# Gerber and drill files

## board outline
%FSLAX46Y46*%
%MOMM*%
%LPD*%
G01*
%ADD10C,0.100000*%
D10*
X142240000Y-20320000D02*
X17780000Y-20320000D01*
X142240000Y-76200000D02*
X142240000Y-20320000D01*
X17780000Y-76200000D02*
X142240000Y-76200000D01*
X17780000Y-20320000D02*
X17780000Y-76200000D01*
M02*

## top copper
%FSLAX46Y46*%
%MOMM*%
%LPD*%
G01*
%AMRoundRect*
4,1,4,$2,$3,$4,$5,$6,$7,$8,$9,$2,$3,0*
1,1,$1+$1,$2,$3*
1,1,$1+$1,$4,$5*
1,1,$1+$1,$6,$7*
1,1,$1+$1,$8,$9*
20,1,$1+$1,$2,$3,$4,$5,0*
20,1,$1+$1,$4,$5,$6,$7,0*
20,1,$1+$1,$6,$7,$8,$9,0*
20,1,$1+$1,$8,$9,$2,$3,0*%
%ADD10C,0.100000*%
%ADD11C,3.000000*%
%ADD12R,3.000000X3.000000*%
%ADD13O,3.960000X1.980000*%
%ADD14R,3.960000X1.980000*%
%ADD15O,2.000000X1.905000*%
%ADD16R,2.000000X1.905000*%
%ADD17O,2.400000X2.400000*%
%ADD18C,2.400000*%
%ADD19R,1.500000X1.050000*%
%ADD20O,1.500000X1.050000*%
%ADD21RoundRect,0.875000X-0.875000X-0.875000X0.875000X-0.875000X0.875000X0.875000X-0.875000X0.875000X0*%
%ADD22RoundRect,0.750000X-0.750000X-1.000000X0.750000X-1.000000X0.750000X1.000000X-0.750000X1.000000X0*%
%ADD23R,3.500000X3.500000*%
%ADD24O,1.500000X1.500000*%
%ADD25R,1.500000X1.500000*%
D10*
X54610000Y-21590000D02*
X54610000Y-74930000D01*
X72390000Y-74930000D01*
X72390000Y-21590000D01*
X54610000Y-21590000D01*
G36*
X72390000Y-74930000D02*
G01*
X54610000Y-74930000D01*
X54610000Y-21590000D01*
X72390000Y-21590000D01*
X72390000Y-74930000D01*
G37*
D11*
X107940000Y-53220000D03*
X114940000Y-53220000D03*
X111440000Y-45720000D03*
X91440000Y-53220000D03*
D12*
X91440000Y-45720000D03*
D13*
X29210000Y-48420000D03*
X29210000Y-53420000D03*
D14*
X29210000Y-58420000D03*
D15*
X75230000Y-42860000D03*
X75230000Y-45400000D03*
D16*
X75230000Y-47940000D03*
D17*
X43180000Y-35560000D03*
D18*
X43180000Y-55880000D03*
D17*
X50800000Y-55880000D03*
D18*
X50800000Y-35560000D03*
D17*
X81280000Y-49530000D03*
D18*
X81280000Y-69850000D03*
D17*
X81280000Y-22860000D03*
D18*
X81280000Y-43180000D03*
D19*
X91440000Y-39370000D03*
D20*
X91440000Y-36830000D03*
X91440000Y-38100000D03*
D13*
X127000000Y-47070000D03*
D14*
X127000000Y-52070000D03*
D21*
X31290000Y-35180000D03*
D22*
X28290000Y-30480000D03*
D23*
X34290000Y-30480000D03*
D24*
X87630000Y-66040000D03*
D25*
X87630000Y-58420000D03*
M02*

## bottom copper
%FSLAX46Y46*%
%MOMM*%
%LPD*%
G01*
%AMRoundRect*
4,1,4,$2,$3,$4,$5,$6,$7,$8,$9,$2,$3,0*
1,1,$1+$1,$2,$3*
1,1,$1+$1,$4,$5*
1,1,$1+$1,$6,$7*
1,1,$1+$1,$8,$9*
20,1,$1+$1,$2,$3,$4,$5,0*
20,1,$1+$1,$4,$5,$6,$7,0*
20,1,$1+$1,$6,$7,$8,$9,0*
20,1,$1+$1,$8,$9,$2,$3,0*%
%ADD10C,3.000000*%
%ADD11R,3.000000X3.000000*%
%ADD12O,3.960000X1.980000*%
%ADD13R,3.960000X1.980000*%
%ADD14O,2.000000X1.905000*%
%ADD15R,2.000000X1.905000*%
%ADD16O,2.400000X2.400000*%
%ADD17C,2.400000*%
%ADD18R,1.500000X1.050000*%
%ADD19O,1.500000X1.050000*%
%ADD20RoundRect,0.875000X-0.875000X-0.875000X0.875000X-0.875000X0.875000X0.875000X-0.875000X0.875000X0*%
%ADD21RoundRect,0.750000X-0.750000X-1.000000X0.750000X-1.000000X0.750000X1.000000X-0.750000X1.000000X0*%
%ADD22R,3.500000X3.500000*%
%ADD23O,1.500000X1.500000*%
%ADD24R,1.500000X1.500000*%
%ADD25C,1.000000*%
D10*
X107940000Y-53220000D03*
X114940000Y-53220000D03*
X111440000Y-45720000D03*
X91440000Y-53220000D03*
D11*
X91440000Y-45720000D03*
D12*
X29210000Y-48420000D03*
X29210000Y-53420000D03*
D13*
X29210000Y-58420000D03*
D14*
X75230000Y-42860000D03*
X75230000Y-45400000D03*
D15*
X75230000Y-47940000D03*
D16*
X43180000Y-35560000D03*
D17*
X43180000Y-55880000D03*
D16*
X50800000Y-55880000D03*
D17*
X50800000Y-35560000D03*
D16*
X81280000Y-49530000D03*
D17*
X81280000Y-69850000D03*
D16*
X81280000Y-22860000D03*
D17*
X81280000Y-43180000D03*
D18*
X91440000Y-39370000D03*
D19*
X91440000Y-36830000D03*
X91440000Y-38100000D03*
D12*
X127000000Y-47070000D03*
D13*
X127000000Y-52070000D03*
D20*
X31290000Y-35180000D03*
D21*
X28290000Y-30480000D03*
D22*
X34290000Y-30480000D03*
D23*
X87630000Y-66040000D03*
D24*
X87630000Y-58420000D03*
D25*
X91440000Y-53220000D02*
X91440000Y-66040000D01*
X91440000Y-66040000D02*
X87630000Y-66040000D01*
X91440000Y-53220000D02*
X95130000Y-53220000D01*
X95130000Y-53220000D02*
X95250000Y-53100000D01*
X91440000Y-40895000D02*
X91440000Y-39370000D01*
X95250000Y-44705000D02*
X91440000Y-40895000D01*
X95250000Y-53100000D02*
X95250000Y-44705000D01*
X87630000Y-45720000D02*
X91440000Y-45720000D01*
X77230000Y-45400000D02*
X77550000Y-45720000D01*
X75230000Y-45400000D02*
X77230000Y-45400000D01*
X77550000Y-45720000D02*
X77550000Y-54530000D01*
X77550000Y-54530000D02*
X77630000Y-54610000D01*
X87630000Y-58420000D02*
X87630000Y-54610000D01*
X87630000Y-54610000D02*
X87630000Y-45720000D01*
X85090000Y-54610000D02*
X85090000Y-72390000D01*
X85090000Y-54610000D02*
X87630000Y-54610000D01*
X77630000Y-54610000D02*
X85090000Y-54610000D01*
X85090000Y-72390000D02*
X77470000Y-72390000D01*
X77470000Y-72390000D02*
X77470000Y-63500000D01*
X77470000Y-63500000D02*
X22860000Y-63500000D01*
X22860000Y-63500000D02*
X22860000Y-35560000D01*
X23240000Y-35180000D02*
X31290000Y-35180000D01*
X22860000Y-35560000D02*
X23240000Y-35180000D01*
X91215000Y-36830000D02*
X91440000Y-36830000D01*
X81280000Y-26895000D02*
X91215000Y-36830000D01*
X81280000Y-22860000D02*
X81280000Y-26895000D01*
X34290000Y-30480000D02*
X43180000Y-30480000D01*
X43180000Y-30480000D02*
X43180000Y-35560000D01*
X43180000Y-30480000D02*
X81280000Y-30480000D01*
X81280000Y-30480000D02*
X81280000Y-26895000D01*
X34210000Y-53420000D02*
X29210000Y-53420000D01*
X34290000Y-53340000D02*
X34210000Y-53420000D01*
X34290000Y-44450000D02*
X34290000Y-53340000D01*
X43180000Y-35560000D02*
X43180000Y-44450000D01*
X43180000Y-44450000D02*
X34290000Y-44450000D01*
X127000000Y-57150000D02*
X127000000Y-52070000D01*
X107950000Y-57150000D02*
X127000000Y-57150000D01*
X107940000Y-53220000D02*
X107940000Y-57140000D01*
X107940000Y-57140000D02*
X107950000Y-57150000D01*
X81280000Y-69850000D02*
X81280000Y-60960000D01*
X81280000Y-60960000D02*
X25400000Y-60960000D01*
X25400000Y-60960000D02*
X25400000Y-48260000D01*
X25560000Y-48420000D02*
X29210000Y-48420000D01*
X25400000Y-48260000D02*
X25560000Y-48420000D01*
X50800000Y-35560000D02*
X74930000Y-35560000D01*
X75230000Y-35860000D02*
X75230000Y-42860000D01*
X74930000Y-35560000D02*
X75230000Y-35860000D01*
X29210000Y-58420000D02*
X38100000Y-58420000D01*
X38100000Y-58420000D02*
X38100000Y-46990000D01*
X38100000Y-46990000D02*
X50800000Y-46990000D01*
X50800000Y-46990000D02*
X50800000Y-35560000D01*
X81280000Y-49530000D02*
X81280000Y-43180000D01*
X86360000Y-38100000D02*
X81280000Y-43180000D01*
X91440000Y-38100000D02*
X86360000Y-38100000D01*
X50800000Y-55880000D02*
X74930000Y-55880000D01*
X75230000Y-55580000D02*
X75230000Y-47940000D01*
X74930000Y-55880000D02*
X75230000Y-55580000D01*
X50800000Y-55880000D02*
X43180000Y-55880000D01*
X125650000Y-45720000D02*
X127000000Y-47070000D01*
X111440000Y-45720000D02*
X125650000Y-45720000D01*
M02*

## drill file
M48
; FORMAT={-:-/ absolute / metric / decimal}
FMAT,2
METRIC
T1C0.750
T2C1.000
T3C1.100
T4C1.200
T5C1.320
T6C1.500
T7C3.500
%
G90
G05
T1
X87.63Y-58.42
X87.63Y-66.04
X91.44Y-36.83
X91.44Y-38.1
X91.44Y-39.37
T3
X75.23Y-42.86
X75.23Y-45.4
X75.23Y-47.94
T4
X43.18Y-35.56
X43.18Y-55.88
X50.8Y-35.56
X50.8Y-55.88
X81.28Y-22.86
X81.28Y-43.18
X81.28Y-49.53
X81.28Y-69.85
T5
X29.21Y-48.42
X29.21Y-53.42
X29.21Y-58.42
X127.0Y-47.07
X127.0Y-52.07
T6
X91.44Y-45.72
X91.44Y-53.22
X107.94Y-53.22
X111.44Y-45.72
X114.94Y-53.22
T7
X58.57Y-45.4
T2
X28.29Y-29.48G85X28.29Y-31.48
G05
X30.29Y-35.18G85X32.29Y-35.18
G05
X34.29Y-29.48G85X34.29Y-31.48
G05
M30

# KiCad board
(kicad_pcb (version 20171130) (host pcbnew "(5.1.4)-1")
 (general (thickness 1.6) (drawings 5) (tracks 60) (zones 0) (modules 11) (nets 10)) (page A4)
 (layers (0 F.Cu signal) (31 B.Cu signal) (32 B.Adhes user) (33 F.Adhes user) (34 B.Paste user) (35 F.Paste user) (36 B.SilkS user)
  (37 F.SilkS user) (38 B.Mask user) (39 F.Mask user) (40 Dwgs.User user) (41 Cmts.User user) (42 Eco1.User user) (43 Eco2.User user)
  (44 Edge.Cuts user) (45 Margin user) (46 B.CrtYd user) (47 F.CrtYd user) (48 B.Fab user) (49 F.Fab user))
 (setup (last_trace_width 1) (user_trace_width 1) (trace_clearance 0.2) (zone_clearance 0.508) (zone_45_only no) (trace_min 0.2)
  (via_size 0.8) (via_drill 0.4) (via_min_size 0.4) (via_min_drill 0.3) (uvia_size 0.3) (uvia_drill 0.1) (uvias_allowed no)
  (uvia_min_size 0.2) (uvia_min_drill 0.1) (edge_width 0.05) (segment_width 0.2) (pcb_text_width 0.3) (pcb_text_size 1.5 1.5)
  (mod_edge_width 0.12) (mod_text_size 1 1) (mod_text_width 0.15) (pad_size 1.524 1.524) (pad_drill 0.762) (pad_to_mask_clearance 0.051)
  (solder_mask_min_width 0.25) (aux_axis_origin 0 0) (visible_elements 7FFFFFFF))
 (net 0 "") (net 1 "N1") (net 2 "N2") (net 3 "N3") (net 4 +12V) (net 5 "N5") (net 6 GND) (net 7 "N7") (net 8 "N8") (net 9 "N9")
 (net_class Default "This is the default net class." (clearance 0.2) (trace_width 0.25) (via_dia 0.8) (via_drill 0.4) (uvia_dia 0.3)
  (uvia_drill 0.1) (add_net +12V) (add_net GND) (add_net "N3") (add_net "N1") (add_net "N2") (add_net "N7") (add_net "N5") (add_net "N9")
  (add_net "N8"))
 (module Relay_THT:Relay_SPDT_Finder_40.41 (layer F.Cu) (at 91.44 45.72)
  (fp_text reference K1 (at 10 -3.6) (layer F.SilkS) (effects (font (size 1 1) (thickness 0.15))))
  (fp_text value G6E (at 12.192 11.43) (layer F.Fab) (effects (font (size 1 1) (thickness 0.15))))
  (pad 12 thru_hole circle (at 16.5 7.5) (size 3 3) (drill 1.5) (layers *.Cu *.Mask) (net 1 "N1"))
  (pad 14 thru_hole circle (at 23.5 7.5) (size 3 3) (drill 1.5) (layers *.Cu *.Mask))
  (pad 11 thru_hole circle (at 20 0) (size 3 3) (drill 1.5) (layers *.Cu *.Mask) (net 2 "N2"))
  (pad A2 thru_hole circle (at 0 7.5) (size 3 3) (drill 1.5) (layers *.Cu *.Mask) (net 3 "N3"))
  (pad A1 thru_hole rect (at 0 0) (size 3 3) (drill 1.5) (layers *.Cu *.Mask) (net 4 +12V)))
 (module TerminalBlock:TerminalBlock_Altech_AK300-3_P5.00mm (layer F.Cu) (at 29.21 58.42 90)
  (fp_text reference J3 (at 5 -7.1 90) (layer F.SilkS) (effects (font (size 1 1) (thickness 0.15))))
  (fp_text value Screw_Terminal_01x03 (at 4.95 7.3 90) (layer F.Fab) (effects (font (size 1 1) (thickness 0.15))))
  (pad 3 thru_hole oval (at 10 0 90) (size 1.98 3.96) (drill 1.32) (layers *.Cu *.Mask) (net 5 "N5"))
  (pad 2 thru_hole oval (at 5 0 90) (size 1.98 3.96) (drill 1.32) (layers *.Cu *.Mask) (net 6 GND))
  (pad 1 thru_hole rect (at 0 0 90) (size 1.98 3.96) (drill 1.32) (layers *.Cu *.Mask) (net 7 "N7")))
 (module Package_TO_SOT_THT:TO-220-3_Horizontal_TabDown (layer F.Cu) (at 75.23 47.94 90)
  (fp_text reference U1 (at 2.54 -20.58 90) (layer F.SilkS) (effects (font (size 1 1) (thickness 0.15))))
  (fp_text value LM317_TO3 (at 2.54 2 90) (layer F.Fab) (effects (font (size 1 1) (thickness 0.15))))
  (pad 3 thru_hole oval (at 5.08 0 90) (size 1.905 2) (drill 1.1) (layers *.Cu *.Mask) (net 7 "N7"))
  (pad 2 thru_hole oval (at 2.54 0 90) (size 1.905 2) (drill 1.1) (layers *.Cu *.Mask) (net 4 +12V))
  (pad 1 thru_hole rect (at 0 0 90) (size 1.905 2) (drill 1.1) (layers *.Cu *.Mask) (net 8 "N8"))
  (pad "" np_thru_hole oval (at 2.54 -16.66 90) (size 3.5 3.5) (drill 3.5) (layers *.Cu *.Mask)))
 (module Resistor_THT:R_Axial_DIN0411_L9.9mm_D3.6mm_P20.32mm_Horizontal (layer F.Cu) (at 43.18 55.88 90)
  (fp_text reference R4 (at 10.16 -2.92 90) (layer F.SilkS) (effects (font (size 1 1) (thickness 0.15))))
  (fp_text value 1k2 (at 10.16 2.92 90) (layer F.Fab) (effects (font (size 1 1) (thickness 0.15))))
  (pad 2 thru_hole oval (at 20.32 0 90) (size 2.4 2.4) (drill 1.2) (layers *.Cu *.Mask) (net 6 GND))
  (pad 1 thru_hole circle (at 0 0 90) (size 2.4 2.4) (drill 1.2) (layers *.Cu *.Mask) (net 8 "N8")))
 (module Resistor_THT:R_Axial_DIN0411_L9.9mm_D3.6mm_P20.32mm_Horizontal (layer F.Cu) (at 50.8 35.56 270)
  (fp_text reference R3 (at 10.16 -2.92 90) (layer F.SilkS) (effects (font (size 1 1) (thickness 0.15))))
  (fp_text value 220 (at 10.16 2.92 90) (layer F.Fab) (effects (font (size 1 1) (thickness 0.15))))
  (pad 2 thru_hole oval (at 20.32 0 270) (size 2.4 2.4) (drill 1.2) (layers *.Cu *.Mask) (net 8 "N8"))
  (pad 1 thru_hole circle (at 0 0 270) (size 2.4 2.4) (drill 1.2) (layers *.Cu *.Mask) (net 7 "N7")))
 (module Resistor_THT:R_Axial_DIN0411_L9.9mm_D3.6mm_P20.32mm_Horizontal (layer F.Cu) (at 81.28 69.85 90)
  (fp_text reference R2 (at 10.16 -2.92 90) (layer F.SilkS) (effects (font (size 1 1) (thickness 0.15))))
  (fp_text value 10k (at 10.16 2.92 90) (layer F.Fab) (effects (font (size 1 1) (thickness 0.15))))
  (pad 2 thru_hole oval (at 20.32 0 90) (size 2.4 2.4) (drill 1.2) (layers *.Cu *.Mask) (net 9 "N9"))
  (pad 1 thru_hole circle (at 0 0 90) (size 2.4 2.4) (drill 1.2) (layers *.Cu *.Mask) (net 5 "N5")))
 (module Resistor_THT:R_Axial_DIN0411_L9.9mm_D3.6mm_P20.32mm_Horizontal (layer F.Cu) (at 81.28 43.18 90)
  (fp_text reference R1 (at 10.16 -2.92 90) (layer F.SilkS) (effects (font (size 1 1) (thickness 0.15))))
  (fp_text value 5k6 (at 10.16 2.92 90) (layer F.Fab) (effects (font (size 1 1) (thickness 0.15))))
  (pad 2 thru_hole oval (at 20.32 0 90) (size 2.4 2.4) (drill 1.2) (layers *.Cu *.Mask) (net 6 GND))
  (pad 1 thru_hole circle (at 0 0 90) (size 2.4 2.4) (drill 1.2) (layers *.Cu *.Mask) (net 9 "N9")))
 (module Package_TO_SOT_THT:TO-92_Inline (layer F.Cu) (at 91.44 39.37 90)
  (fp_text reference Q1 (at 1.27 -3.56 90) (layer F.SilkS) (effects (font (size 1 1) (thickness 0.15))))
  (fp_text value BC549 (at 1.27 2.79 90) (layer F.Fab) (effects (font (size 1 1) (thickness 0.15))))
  (pad 1 thru_hole rect (at 0 0 90) (size 1.05 1.5) (drill 0.75) (layers *.Cu *.Mask) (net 3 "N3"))
  (pad 3 thru_hole oval (at 2.54 0 90) (size 1.05 1.5) (drill 0.75) (layers *.Cu *.Mask) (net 6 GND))
  (pad 2 thru_hole oval (at 1.27 0 90) (size 1.05 1.5) (drill 0.75) (layers *.Cu *.Mask) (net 9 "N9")))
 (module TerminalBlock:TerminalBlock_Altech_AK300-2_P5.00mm (layer F.Cu) (at 127 52.07 90)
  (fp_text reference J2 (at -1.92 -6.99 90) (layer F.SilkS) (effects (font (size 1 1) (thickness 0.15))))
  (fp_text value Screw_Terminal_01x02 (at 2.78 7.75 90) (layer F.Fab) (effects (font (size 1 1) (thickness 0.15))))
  (pad 2 thru_hole oval (at 5 0 90) (size 1.98 3.96) (drill 1.32) (layers *.Cu *.Mask) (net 2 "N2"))
  (pad 1 thru_hole rect (at 0 0 90) (size 1.98 3.96) (drill 1.32) (layers *.Cu *.Mask) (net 1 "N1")))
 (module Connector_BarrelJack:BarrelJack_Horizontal (layer F.Cu) (at 34.29 30.48)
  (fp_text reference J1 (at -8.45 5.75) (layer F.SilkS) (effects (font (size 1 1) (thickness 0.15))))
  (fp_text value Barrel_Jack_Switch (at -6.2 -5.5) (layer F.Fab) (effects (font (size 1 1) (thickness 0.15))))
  (pad 3 thru_hole roundrect (at -3 4.7) (size 3.5 3.5) (drill oval 3 1) (layers *.Cu *.Mask) (roundrect_rratio 0.25) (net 4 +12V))
  (pad 2 thru_hole roundrect (at -6 0) (size 3 3.5) (drill oval 1 3) (layers *.Cu *.Mask) (roundrect_rratio 0.25))
  (pad 1 thru_hole rect (at 0 0) (size 3.5 3.5) (drill oval 1 3) (layers *.Cu *.Mask) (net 6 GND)))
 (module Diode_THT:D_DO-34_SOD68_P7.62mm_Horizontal (layer F.Cu) (at 87.63 58.42 270)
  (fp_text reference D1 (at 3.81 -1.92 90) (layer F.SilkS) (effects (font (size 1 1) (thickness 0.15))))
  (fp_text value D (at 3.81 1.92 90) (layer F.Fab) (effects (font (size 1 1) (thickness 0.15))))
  (pad 2 thru_hole oval (at 7.62 0 270) (size 1.5 1.5) (drill 0.75) (layers *.Cu *.Mask) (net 3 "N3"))
  (pad 1 thru_hole rect (at 0 0 270) (size 1.5 1.5) (drill 0.75) (layers *.Cu *.Mask) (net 4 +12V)))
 (gr_poly (pts (xy 54.61 21.59) (xy 54.61 74.93) (xy 72.39 74.93) (xy 72.39 21.59)) (layer F.Cu) (width 0.1))
 (gr_line (start 142.24 20.32) (end 17.78 20.32) (layer Edge.Cuts) (width 0.1))
 (gr_line (start 142.24 76.2) (end 142.24 20.32) (layer Edge.Cuts) (width 0.1))
 (gr_line (start 17.78 76.2) (end 142.24 76.2) (layer Edge.Cuts) (width 0.1))
 (gr_line (start 17.78 20.32) (end 17.78 76.2) (layer Edge.Cuts) (width 0.1))
 (segment (start 91.44 53.22) (end 91.44 66.04) (width 1) (layer B.Cu) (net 3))
 (segment (start 91.44 66.04) (end 87.63 66.04) (width 1) (layer B.Cu) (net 3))
 (segment (start 91.44 53.22) (end 95.13 53.22) (width 1) (layer B.Cu) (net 3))
 (segment (start 95.13 53.22) (end 95.25 53.1) (width 1) (layer B.Cu) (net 3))
 (segment (start 91.44 40.895) (end 91.44 39.37) (width 1) (layer B.Cu) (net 3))
 (segment (start 95.25 44.705) (end 91.44 40.895) (width 1) (layer B.Cu) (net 3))
 (segment (start 95.25 53.1) (end 95.25 44.705) (width 1) (layer B.Cu) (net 3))
 (segment (start 87.63 45.72) (end 91.44 45.72) (width 1) (layer B.Cu) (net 4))
 (segment (start 77.23 45.4) (end 77.55 45.72) (width 1) (layer B.Cu) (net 4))
 (segment (start 75.23 45.4) (end 77.23 45.4) (width 1) (layer B.Cu) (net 4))
 (segment (start 77.55 45.72) (end 77.55 54.53) (width 1) (layer B.Cu) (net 4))
 (segment (start 77.55 54.53) (end 77.63 54.61) (width 1) (layer B.Cu) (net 4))
 (segment (start 87.63 58.42) (end 87.63 54.61) (width 1) (layer B.Cu) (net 4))
 (segment (start 87.63 54.61) (end 87.63 45.72) (width 1) (layer B.Cu) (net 4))
 (segment (start 85.09 54.61) (end 85.09 72.39) (width 1) (layer B.Cu) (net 4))
 (segment (start 85.09 54.61) (end 87.63 54.61) (width 1) (layer B.Cu) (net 4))
 (segment (start 77.63 54.61) (end 85.09 54.61) (width 1) (layer B.Cu) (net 4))
 (segment (start 85.09 72.39) (end 77.47 72.39) (width 1) (layer B.Cu) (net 4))
 (segment (start 77.47 72.39) (end 77.47 63.5) (width 1) (layer B.Cu) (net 4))
 (segment (start 77.47 63.5) (end 22.86 63.5) (width 1) (layer B.Cu) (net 4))
 (segment (start 22.86 63.5) (end 22.86 35.56) (width 1) (layer B.Cu) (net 4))
 (segment (start 23.24 35.18) (end 31.29 35.18) (width 1) (layer B.Cu) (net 4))
 (segment (start 22.86 35.56) (end 23.24 35.18) (width 1) (layer B.Cu) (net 4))
 (segment (start 91.215 36.83) (end 91.44 36.83) (width 1) (layer B.Cu) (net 6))
 (segment (start 81.28 26.895) (end 91.215 36.83) (width 1) (layer B.Cu) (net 6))
 (segment (start 81.28 22.86) (end 81.28 26.895) (width 1) (layer B.Cu) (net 6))
 (segment (start 34.29 30.48) (end 43.18 30.48) (width 1) (layer B.Cu) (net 6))
 (segment (start 43.18 30.48) (end 43.18 35.56) (width 1) (layer B.Cu) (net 6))
 (segment (start 43.18 30.48) (end 81.28 30.48) (width 1) (layer B.Cu) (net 6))
 (segment (start 81.28 30.48) (end 81.28 26.895) (width 1) (layer B.Cu) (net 6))
 (segment (start 34.21 53.42) (end 29.21 53.42) (width 1) (layer B.Cu) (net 6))
 (segment (start 34.29 53.34) (end 34.21 53.42) (width 1) (layer B.Cu) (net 6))
 (segment (start 34.29 44.45) (end 34.29 53.34) (width 1) (layer B.Cu) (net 6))
 (segment (start 43.18 35.56) (end 43.18 44.45) (width 1) (layer B.Cu) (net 6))
 (segment (start 43.18 44.45) (end 34.29 44.45) (width 1) (layer B.Cu) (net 6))
 (segment (start 127 57.15) (end 127 52.07) (width 1) (layer B.Cu) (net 1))
 (segment (start 107.95 57.15) (end 127 57.15) (width 1) (layer B.Cu) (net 1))
 (segment (start 107.94 53.22) (end 107.94 57.14) (width 1) (layer B.Cu) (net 1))
 (segment (start 107.94 57.14) (end 107.95 57.15) (width 1) (layer B.Cu) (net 1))
 (segment (start 81.28 69.85) (end 81.28 60.96) (width 1) (layer B.Cu) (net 5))
 (segment (start 81.28 60.96) (end 25.4 60.96) (width 1) (layer B.Cu) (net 5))
 (segment (start 25.4 60.96) (end 25.4 48.26) (width 1) (layer B.Cu) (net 5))
 (segment (start 25.56 48.42) (end 29.21 48.42) (width 1) (layer B.Cu) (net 5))
 (segment (start 25.4 48.26) (end 25.56 48.42) (width 1) (layer B.Cu) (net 5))
 (segment (start 50.8 35.56) (end 74.93 35.56) (width 1) (layer B.Cu) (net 7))
 (segment (start 75.23 35.86) (end 75.23 42.86) (width 1) (layer B.Cu) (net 7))
 (segment (start 74.93 35.56) (end 75.23 35.86) (width 1) (layer B.Cu) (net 7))
 (segment (start 29.21 58.42) (end 38.1 58.42) (width 1) (layer B.Cu) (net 7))
 (segment (start 38.1 58.42) (end 38.1 46.99) (width 1) (layer B.Cu) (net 7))
 (segment (start 38.1 46.99) (end 50.8 46.99) (width 1) (layer B.Cu) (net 7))
 (segment (start 50.8 46.99) (end 50.8 35.56) (width 1) (layer B.Cu) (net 7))
 (segment (start 81.28 49.53) (end 81.28 43.18) (width 1) (layer B.Cu) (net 9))
 (segment (start 86.36 38.1) (end 81.28 43.18) (width 1) (layer B.Cu) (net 9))
 (segment (start 91.44 38.1) (end 86.36 38.1) (width 1) (layer B.Cu) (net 9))
 (segment (start 50.8 55.88) (end 74.93 55.88) (width 1) (layer B.Cu) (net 8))
 (segment (start 75.23 55.58) (end 75.23 47.94) (width 1) (layer B.Cu) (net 8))
 (segment (start 74.93 55.88) (end 75.23 55.58) (width 1) (layer B.Cu) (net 8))
 (segment (start 50.8 55.88) (end 43.18 55.88) (width 1) (layer B.Cu) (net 8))
 (segment (start 125.65 45.72) (end 127 47.07) (width 1) (layer B.Cu) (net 2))
 (segment (start 111.44 45.72) (end 125.65 45.72) (width 1) (layer B.Cu) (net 2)))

